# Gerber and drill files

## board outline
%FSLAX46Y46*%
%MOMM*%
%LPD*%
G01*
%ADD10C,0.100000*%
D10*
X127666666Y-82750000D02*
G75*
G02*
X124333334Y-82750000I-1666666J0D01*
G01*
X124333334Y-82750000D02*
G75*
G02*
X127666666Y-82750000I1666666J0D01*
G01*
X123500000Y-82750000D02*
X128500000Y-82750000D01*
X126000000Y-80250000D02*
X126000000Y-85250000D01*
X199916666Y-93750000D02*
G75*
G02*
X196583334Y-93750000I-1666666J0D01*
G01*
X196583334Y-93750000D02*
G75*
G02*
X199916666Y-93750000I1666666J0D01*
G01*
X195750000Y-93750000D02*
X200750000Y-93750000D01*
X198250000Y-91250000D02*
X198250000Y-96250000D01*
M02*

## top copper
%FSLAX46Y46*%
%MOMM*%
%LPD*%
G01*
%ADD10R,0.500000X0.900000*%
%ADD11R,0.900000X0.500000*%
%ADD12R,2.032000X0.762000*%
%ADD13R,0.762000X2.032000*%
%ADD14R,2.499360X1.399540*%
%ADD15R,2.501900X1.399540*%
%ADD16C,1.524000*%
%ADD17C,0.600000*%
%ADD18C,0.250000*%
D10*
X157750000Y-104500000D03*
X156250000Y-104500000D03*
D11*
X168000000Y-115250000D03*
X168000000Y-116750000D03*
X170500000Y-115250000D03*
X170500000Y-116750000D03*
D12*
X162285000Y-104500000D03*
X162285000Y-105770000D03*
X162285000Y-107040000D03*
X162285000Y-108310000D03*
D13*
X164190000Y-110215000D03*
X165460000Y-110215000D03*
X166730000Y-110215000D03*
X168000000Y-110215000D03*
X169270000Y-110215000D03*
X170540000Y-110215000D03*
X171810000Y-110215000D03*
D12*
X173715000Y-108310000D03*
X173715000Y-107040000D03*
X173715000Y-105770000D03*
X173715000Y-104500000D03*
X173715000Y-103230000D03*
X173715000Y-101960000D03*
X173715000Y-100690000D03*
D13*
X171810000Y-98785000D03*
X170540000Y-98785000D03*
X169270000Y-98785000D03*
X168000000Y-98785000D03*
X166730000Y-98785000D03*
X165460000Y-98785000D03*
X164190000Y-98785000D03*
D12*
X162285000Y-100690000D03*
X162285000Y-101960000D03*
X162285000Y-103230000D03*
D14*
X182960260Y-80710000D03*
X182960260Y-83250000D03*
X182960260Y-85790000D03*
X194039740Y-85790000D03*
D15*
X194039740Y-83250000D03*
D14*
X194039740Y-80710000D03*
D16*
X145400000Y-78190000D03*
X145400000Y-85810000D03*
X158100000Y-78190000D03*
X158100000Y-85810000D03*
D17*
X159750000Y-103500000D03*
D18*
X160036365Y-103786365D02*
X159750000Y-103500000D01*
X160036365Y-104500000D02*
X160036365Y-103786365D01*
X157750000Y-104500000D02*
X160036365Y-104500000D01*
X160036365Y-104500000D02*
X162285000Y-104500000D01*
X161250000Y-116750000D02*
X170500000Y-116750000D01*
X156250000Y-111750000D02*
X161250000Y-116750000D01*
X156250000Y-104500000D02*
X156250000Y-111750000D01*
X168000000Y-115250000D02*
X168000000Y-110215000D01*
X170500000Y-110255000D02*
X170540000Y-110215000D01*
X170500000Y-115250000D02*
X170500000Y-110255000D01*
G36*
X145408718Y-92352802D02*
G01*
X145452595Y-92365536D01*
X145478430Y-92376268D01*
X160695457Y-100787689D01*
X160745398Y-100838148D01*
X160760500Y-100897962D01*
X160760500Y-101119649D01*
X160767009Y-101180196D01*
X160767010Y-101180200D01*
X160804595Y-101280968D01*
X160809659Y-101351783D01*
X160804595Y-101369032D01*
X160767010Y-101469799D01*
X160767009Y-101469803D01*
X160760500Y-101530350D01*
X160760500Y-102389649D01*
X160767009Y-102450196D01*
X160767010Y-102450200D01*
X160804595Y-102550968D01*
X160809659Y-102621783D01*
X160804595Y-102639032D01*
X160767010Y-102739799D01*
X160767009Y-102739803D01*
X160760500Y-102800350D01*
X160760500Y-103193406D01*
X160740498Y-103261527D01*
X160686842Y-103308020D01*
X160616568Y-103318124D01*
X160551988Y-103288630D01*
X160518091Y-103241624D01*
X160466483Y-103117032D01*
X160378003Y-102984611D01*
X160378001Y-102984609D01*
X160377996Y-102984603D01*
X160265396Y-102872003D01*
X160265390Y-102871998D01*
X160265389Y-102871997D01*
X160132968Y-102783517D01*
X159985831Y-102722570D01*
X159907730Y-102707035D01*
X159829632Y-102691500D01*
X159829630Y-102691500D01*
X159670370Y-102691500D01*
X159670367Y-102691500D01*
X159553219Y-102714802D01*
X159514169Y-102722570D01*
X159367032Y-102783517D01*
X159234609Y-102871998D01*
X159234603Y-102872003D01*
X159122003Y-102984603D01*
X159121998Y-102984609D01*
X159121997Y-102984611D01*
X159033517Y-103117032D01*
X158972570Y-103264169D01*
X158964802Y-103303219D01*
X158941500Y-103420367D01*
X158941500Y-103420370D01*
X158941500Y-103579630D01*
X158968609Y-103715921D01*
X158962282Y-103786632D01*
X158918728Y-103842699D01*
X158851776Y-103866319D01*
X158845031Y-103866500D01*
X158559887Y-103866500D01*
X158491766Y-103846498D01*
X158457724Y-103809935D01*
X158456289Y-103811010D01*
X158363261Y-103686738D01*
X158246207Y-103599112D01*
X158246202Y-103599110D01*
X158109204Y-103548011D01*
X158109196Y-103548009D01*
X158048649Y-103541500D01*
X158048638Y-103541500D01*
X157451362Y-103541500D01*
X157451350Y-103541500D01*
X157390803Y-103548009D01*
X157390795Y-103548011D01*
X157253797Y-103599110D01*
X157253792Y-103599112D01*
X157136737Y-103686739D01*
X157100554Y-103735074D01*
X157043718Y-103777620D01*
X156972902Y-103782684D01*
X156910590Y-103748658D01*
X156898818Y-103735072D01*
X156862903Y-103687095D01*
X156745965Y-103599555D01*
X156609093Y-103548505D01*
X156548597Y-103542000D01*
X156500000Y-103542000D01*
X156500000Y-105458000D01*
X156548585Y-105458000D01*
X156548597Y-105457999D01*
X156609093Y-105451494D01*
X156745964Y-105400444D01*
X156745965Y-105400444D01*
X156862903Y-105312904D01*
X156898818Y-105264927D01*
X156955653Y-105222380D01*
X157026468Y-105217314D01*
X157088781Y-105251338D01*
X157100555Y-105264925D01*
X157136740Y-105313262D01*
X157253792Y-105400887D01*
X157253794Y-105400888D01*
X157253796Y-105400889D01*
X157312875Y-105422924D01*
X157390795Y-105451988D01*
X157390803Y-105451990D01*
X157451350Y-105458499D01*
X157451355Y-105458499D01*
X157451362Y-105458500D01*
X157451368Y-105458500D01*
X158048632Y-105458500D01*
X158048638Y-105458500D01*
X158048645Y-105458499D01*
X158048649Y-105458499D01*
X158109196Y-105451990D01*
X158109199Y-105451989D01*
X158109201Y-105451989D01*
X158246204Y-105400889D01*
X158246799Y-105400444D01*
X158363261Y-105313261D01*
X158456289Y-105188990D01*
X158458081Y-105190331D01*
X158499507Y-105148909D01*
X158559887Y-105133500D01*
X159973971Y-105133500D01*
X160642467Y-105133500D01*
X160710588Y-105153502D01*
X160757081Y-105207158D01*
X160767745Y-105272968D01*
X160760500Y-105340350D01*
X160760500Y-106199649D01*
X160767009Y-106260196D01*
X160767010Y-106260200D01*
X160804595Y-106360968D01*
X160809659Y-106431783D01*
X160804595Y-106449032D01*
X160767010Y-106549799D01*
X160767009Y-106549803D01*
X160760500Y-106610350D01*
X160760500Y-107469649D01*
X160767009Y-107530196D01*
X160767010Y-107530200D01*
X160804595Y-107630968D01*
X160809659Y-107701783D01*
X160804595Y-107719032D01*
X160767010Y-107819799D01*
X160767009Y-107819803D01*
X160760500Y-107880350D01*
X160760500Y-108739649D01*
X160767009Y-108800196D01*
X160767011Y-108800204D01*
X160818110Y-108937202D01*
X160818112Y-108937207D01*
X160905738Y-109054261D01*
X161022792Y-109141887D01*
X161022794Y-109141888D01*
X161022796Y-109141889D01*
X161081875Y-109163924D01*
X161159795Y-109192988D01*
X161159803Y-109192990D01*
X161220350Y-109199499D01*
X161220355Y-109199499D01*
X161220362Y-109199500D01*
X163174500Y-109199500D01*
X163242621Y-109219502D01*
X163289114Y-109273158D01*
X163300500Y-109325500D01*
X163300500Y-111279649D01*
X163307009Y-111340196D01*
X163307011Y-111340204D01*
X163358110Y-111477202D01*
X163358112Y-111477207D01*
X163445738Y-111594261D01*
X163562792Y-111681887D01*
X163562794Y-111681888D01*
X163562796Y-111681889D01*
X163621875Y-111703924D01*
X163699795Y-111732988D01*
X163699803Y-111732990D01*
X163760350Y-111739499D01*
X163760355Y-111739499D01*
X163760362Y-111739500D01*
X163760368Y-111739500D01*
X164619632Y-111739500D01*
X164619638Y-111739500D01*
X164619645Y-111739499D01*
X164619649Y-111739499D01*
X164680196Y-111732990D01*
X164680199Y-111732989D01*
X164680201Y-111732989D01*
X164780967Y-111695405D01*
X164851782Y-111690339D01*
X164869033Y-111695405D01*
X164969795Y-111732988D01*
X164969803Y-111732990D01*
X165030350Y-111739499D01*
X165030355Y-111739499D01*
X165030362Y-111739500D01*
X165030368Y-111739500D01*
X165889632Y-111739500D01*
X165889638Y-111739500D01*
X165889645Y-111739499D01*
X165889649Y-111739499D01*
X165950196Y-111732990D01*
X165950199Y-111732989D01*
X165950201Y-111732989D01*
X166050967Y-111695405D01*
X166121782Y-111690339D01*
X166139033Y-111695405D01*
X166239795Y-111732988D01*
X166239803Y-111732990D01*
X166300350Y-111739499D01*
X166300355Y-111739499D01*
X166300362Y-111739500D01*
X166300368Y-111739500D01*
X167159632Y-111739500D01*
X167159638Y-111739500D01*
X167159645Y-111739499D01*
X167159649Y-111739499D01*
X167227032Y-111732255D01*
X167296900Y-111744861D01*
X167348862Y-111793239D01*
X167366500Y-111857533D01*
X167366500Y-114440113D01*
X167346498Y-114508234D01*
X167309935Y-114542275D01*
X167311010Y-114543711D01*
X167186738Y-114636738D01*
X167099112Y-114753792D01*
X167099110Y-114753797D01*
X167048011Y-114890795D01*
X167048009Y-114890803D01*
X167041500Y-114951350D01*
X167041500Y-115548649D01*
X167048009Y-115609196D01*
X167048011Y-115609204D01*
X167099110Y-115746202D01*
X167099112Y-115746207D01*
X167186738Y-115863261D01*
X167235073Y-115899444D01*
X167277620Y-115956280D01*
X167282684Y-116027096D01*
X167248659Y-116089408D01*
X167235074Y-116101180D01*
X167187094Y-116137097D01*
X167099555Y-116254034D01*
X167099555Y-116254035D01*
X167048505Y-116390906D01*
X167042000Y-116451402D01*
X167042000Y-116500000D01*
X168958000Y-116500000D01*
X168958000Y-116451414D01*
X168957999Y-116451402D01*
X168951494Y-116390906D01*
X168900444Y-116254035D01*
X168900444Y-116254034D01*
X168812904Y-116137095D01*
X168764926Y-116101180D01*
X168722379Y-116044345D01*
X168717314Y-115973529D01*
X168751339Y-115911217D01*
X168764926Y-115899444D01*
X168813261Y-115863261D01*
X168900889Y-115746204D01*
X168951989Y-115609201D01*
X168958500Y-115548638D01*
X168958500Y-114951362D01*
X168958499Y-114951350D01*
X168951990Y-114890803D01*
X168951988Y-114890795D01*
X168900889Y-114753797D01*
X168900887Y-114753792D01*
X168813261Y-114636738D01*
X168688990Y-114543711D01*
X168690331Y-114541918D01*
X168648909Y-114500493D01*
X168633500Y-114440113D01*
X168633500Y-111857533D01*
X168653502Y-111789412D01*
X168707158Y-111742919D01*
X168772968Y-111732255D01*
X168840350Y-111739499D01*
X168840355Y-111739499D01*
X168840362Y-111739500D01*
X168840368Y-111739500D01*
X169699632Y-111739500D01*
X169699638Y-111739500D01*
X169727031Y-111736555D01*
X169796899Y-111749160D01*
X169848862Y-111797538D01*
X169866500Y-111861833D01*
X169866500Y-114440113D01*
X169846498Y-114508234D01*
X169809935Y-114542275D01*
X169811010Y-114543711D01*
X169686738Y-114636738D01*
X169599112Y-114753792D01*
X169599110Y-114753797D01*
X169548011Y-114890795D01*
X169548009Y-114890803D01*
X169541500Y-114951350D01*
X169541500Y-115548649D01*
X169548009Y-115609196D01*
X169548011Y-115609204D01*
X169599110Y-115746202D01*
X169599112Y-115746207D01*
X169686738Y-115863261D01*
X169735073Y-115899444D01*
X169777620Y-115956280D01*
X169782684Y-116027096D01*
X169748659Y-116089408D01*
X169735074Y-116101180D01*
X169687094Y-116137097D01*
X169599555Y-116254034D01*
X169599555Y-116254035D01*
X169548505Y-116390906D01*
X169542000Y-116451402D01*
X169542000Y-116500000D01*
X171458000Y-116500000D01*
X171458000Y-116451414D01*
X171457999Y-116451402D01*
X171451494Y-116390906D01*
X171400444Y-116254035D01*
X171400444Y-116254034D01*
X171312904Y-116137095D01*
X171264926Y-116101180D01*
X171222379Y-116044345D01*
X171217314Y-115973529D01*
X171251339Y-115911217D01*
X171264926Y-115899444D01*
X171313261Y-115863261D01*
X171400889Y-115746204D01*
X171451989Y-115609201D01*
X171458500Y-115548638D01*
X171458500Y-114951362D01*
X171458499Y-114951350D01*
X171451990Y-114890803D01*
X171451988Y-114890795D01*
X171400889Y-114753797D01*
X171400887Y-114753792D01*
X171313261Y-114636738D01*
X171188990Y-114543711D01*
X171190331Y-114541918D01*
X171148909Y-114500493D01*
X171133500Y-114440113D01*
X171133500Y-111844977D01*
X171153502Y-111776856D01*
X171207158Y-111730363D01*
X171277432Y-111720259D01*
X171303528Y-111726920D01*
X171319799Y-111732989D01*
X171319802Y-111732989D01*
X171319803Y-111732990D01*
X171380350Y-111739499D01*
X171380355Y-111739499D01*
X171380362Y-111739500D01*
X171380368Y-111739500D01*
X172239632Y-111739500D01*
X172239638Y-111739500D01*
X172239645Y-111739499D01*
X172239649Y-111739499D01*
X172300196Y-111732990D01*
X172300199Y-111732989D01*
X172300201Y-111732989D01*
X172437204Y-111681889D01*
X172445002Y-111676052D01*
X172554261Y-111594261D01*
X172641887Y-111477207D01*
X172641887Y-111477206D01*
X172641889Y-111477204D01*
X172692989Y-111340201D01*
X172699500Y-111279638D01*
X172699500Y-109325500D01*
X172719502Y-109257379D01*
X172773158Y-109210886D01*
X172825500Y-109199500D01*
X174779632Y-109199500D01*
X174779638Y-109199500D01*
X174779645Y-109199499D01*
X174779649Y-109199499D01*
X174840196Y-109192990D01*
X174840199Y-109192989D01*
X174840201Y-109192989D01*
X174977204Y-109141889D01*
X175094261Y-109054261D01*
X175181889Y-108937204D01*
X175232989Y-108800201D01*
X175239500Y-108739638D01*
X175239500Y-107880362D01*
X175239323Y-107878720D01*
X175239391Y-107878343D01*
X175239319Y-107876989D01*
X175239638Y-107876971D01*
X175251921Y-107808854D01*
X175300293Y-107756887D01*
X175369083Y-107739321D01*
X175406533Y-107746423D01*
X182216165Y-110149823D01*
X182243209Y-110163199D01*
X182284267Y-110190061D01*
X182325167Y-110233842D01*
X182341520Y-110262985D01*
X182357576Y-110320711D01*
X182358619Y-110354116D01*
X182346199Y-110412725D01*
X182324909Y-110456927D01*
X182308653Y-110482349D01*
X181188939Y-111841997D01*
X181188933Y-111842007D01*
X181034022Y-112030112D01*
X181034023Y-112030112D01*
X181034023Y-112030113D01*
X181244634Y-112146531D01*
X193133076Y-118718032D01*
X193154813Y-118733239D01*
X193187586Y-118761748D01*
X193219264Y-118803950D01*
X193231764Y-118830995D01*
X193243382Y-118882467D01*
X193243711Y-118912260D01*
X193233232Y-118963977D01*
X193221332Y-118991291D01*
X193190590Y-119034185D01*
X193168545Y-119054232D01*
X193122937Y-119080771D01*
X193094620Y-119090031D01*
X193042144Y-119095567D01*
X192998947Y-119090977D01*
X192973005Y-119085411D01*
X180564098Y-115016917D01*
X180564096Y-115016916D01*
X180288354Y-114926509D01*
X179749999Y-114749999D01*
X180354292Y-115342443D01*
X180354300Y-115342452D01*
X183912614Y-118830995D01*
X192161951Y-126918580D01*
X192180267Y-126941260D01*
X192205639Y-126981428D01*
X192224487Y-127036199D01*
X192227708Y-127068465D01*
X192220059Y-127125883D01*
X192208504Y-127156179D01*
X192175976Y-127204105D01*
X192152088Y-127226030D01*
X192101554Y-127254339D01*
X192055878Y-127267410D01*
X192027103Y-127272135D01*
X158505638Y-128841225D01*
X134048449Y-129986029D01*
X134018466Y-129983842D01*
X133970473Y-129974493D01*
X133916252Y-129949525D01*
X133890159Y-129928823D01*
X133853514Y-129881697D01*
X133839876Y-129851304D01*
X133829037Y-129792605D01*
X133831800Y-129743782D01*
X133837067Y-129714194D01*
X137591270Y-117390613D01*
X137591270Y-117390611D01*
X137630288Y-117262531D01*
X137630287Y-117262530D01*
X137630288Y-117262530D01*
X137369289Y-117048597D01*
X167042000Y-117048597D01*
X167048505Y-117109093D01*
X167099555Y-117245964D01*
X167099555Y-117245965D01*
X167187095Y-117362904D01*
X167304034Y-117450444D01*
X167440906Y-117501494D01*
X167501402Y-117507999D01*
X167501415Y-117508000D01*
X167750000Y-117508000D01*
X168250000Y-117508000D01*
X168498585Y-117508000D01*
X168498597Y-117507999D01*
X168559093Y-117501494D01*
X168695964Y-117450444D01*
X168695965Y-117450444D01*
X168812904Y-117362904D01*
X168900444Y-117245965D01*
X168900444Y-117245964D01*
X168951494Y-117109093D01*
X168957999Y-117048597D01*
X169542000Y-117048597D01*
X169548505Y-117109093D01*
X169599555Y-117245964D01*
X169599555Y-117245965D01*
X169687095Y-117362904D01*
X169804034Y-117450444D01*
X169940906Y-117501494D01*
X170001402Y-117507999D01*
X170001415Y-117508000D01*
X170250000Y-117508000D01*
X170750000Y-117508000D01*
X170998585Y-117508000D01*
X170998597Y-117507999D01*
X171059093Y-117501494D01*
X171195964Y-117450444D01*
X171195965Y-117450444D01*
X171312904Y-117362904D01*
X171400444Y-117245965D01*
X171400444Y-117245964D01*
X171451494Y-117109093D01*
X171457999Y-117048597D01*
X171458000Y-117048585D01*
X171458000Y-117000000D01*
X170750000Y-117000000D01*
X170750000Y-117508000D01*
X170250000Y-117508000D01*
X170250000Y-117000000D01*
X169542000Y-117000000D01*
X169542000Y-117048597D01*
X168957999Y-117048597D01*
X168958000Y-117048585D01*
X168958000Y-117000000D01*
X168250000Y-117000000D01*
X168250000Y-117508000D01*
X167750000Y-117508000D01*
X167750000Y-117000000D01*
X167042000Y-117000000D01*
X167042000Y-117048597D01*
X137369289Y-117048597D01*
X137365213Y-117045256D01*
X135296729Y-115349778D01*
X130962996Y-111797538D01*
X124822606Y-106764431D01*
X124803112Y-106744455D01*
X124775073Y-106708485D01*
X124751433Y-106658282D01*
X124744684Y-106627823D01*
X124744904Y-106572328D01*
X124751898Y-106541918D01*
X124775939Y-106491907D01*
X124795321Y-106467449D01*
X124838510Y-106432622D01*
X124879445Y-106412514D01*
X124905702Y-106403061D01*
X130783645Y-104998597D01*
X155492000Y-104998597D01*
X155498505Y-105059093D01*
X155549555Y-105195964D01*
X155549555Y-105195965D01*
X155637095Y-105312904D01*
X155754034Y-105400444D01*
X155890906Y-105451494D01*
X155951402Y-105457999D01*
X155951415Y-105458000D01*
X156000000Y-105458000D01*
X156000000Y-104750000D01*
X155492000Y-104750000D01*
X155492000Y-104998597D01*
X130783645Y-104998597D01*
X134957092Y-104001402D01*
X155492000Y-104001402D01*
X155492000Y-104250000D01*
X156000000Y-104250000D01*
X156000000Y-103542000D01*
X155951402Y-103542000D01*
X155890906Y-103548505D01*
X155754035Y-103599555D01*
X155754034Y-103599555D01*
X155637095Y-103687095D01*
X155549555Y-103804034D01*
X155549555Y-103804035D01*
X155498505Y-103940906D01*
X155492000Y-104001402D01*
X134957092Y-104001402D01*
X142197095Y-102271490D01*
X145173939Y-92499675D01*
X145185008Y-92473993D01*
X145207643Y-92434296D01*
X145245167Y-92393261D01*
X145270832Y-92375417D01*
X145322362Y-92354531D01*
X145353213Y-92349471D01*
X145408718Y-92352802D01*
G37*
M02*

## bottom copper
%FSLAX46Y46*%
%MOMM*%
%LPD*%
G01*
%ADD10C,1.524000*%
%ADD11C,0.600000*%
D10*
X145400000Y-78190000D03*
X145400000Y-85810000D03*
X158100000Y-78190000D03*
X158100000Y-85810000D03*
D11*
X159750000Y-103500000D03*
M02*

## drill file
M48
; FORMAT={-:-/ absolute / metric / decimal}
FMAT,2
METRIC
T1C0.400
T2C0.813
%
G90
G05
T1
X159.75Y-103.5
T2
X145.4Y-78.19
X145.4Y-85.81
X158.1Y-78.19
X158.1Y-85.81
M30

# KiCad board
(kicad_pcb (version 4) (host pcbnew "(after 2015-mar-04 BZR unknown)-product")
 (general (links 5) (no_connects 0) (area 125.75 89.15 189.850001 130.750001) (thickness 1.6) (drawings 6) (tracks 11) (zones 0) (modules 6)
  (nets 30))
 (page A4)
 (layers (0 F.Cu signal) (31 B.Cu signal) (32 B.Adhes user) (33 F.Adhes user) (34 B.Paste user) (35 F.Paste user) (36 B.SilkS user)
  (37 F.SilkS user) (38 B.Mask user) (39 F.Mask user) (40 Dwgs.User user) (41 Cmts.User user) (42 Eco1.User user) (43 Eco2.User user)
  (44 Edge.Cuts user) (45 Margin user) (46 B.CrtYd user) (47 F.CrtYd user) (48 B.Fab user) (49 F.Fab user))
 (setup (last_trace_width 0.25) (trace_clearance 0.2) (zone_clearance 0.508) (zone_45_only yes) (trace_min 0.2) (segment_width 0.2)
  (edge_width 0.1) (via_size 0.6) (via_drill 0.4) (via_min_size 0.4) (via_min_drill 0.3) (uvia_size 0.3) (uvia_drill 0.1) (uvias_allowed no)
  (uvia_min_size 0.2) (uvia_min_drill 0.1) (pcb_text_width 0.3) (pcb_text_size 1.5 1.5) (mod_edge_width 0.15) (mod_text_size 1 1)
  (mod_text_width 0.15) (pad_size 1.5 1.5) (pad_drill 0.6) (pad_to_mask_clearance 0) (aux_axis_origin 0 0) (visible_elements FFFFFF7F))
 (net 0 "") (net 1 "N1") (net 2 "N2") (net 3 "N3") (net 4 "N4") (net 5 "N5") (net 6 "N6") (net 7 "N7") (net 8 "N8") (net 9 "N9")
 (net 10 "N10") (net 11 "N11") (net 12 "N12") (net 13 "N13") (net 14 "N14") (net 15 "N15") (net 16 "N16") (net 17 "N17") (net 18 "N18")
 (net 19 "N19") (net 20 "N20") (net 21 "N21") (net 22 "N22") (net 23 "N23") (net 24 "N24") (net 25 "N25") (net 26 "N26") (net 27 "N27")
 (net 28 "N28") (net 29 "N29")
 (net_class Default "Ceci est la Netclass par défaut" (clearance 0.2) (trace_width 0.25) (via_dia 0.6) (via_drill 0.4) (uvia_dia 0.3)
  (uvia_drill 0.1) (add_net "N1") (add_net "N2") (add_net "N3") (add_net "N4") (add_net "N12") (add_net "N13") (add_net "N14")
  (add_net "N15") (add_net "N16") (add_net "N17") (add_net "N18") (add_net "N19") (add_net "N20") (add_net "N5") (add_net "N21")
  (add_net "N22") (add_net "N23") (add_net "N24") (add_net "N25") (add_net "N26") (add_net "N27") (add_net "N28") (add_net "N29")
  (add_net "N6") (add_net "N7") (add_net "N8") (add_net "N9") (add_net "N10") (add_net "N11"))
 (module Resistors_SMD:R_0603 (layer F.Cu) (at 157 104.5 180)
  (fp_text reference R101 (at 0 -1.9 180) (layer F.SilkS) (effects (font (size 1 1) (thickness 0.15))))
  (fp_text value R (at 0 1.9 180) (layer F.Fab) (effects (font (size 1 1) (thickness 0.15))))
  (pad 1 smd rect (at -0.75 0 180) (size 0.5 0.9) (layers F.Cu F.Paste F.Mask) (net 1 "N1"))
  (pad 2 smd rect (at 0.75 0 180) (size 0.5 0.9) (layers F.Cu F.Paste F.Mask) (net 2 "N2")))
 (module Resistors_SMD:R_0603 (layer F.Cu) (at 168 116 270)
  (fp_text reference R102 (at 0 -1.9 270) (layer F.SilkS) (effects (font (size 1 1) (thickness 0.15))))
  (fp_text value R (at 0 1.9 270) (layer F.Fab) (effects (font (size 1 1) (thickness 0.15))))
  (pad 1 smd rect (at -0.75 0 270) (size 0.5 0.9) (layers F.Cu F.Paste F.Mask) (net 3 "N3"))
  (pad 2 smd rect (at 0.75 0 270) (size 0.5 0.9) (layers F.Cu F.Paste F.Mask) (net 2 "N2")))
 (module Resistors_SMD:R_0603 (layer F.Cu) (at 170.5 116 270)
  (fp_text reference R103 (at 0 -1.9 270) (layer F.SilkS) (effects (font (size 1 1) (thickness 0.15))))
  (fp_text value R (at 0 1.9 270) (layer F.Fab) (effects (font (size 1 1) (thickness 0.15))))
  (pad 1 smd rect (at -0.75 0 270) (size 0.5 0.9) (layers F.Cu F.Paste F.Mask) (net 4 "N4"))
  (pad 2 smd rect (at 0.75 0 270) (size 0.5 0.9) (layers F.Cu F.Paste F.Mask) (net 2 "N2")))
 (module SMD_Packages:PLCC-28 (layer F.Cu) (at 168 104.5)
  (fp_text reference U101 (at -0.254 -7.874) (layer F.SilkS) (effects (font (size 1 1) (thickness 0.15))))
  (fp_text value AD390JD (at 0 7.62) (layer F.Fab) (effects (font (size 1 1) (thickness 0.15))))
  (pad 1 smd rect (at -5.715 0) (size 2.032 0.762) (layers F.Cu F.Paste F.Mask) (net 1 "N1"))
  (pad 2 smd rect (at -5.715 1.27) (size 2.032 0.762) (layers F.Cu F.Paste F.Mask) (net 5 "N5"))
  (pad 3 smd rect (at -5.715 2.54) (size 2.032 0.762) (layers F.Cu F.Paste F.Mask) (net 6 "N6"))
  (pad 4 smd rect (at -5.715 3.81) (size 2.032 0.762) (layers F.Cu F.Paste F.Mask) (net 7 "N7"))
  (pad 5 smd rect (at -3.81 5.715) (size 0.762 2.032) (layers F.Cu F.Paste F.Mask) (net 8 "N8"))
  (pad 6 smd rect (at -2.54 5.715) (size 0.762 2.032) (layers F.Cu F.Paste F.Mask) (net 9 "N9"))
  (pad 7 smd rect (at -1.27 5.715) (size 0.762 2.032) (layers F.Cu F.Paste F.Mask) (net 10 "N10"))
  (pad 8 smd rect (at 0 5.715) (size 0.762 2.032) (layers F.Cu F.Paste F.Mask) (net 3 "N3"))
  (pad 9 smd rect (at 1.27 5.715) (size 0.762 2.032) (layers F.Cu F.Paste F.Mask) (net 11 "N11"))
  (pad 10 smd rect (at 2.54 5.715) (size 0.762 2.032) (layers F.Cu F.Paste F.Mask) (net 4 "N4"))
  (pad 11 smd rect (at 3.81 5.715) (size 0.762 2.032) (layers F.Cu F.Paste F.Mask) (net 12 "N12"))
  (pad 12 smd rect (at 5.715 3.81) (size 2.032 0.762) (layers F.Cu F.Paste F.Mask) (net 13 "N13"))
  (pad 13 smd rect (at 5.715 2.54) (size 2.032 0.762) (layers F.Cu F.Paste F.Mask) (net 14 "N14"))
  (pad 14 smd rect (at 5.715 1.27) (size 2.032 0.762) (layers F.Cu F.Paste F.Mask) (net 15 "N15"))
  (pad 15 smd rect (at 5.715 0) (size 2.032 0.762) (layers F.Cu F.Paste F.Mask) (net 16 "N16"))
  (pad 16 smd rect (at 5.715 -1.27) (size 2.032 0.762) (layers F.Cu F.Paste F.Mask) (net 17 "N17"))
  (pad 17 smd rect (at 5.715 -2.54) (size 2.032 0.762) (layers F.Cu F.Paste F.Mask) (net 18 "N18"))
  (pad 18 smd rect (at 5.715 -3.81) (size 2.032 0.762) (layers F.Cu F.Paste F.Mask) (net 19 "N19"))
  (pad 19 smd rect (at 3.81 -5.715) (size 0.762 2.032) (layers F.Cu F.Paste F.Mask) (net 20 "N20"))
  (pad 20 smd rect (at 2.54 -5.715) (size 0.762 2.032) (layers F.Cu F.Paste F.Mask) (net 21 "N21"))
  (pad 21 smd rect (at 1.27 -5.715) (size 0.762 2.032) (layers F.Cu F.Paste F.Mask) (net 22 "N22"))
  (pad 22 smd rect (at 0 -5.715) (size 0.762 2.032) (layers F.Cu F.Paste F.Mask) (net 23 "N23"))
  (pad 23 smd rect (at -1.27 -5.715) (size 0.762 2.032) (layers F.Cu F.Paste F.Mask) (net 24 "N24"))
  (pad 24 smd rect (at -2.54 -5.715) (size 0.762 2.032) (layers F.Cu F.Paste F.Mask) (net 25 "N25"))
  (pad 25 smd rect (at -3.81 -5.715) (size 0.762 2.032) (layers F.Cu F.Paste F.Mask) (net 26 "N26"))
  (pad 26 smd rect (at -5.715 -3.81) (size 2.032 0.762) (layers F.Cu F.Paste F.Mask) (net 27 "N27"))
  (pad 27 smd rect (at -5.715 -2.54) (size 2.032 0.762) (layers F.Cu F.Paste F.Mask) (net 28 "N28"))
  (pad 28 smd rect (at -5.715 -1.27) (size 2.032 0.762) (layers F.Cu F.Paste F.Mask) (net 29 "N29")))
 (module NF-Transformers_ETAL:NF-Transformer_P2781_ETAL (layer F.Cu) (at 188.5 83.25)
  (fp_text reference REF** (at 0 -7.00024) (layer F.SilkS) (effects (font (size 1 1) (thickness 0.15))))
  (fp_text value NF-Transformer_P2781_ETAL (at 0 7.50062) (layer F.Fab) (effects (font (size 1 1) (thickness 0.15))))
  (pad 1 smd rect (at -5.53974 -2.54) (size 2.49936 1.39954) (layers F.Cu F.Paste F.Mask))
  (pad 2 smd rect (at -5.53974 0) (size 2.49936 1.39954) (layers F.Cu F.Paste F.Mask))
  (pad 3 smd rect (at -5.53974 2.54) (size 2.49936 1.39954) (layers F.Cu F.Paste F.Mask))
  (pad 4 smd rect (at 5.53974 2.54) (size 2.49936 1.39954) (layers F.Cu F.Paste F.Mask))
  (pad 5 smd rect (at 5.53974 0) (size 2.5019 1.39954) (layers F.Cu F.Paste F.Mask))
  (pad 6 smd rect (at 5.53974 -2.54) (size 2.49936 1.39954) (layers F.Cu F.Paste F.Mask))
  (pad 7 smd oval (at -1.99898 0 90) (size 3.50012 1.39954) (layers F.Adhes))
  (pad 7 smd oval (at 1.99898 0 90) (size 3.50012 1.39954) (layers F.Adhes)))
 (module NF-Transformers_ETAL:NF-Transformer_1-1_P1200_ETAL (layer F.Cu) (at 151.75 82)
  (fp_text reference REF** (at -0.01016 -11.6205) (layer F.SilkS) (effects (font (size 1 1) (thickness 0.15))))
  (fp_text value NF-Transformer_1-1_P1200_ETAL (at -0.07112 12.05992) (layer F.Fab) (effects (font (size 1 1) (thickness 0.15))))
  (pad 6 thru_hole circle (at -6.35 -3.81) (size 1.524 1.524) (drill 0.8128) (layers *.Cu *.Mask F.SilkS))
  (pad 4 thru_hole circle (at -6.35 3.81) (size 1.524 1.524) (drill 0.8128) (layers *.Cu *.Mask F.SilkS))
  (pad 1 thru_hole circle (at 6.35 -3.81) (size 1.524 1.524) (drill 0.8128) (layers *.Cu *.Mask F.SilkS))
  (pad 3 thru_hole circle (at 6.35 3.81) (size 1.524 1.524) (drill 0.8128) (layers *.Cu *.Mask F.SilkS)))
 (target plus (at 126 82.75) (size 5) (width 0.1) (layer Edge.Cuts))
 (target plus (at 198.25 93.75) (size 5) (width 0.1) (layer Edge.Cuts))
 (via (at 159.75 103.5) (size 0.6) (drill 0.4) (layers F.Cu B.Cu) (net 1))
 (segment (start 160.036365 103.786365) (end 159.75 103.5) (width 0.25) (layer F.Cu) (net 1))
 (segment (start 160.036365 104.5) (end 160.036365 103.786365) (width 0.25) (layer F.Cu) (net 1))
 (segment (start 157.75 104.5) (end 160.036365 104.5) (width 0.25) (layer F.Cu) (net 1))
 (segment (start 160.036365 104.5) (end 162.285 104.5) (width 0.25) (layer F.Cu) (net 1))
 (segment (start 161.25 116.75) (end 170.5 116.75) (width 0.25) (layer F.Cu) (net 2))
 (segment (start 156.25 111.75) (end 161.25 116.75) (width 0.25) (layer F.Cu) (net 2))
 (segment (start 156.25 104.5) (end 156.25 111.75) (width 0.25) (layer F.Cu) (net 2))
 (segment (start 168 115.25) (end 168 110.215) (width 0.25) (layer F.Cu) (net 3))
 (segment (start 170.5 110.255) (end 170.54 110.215) (width 0.25) (layer F.Cu) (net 4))
 (segment (start 170.5 115.25) (end 170.5 110.255) (width 0.25) (layer F.Cu) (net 4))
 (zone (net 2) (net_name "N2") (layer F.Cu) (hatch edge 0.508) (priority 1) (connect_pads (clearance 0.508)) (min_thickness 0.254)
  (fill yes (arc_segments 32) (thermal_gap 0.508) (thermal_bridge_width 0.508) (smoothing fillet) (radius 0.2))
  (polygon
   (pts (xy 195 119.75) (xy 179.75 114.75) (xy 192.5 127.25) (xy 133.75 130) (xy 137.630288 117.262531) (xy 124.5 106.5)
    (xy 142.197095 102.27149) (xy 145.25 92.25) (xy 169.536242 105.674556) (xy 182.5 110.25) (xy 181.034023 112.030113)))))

